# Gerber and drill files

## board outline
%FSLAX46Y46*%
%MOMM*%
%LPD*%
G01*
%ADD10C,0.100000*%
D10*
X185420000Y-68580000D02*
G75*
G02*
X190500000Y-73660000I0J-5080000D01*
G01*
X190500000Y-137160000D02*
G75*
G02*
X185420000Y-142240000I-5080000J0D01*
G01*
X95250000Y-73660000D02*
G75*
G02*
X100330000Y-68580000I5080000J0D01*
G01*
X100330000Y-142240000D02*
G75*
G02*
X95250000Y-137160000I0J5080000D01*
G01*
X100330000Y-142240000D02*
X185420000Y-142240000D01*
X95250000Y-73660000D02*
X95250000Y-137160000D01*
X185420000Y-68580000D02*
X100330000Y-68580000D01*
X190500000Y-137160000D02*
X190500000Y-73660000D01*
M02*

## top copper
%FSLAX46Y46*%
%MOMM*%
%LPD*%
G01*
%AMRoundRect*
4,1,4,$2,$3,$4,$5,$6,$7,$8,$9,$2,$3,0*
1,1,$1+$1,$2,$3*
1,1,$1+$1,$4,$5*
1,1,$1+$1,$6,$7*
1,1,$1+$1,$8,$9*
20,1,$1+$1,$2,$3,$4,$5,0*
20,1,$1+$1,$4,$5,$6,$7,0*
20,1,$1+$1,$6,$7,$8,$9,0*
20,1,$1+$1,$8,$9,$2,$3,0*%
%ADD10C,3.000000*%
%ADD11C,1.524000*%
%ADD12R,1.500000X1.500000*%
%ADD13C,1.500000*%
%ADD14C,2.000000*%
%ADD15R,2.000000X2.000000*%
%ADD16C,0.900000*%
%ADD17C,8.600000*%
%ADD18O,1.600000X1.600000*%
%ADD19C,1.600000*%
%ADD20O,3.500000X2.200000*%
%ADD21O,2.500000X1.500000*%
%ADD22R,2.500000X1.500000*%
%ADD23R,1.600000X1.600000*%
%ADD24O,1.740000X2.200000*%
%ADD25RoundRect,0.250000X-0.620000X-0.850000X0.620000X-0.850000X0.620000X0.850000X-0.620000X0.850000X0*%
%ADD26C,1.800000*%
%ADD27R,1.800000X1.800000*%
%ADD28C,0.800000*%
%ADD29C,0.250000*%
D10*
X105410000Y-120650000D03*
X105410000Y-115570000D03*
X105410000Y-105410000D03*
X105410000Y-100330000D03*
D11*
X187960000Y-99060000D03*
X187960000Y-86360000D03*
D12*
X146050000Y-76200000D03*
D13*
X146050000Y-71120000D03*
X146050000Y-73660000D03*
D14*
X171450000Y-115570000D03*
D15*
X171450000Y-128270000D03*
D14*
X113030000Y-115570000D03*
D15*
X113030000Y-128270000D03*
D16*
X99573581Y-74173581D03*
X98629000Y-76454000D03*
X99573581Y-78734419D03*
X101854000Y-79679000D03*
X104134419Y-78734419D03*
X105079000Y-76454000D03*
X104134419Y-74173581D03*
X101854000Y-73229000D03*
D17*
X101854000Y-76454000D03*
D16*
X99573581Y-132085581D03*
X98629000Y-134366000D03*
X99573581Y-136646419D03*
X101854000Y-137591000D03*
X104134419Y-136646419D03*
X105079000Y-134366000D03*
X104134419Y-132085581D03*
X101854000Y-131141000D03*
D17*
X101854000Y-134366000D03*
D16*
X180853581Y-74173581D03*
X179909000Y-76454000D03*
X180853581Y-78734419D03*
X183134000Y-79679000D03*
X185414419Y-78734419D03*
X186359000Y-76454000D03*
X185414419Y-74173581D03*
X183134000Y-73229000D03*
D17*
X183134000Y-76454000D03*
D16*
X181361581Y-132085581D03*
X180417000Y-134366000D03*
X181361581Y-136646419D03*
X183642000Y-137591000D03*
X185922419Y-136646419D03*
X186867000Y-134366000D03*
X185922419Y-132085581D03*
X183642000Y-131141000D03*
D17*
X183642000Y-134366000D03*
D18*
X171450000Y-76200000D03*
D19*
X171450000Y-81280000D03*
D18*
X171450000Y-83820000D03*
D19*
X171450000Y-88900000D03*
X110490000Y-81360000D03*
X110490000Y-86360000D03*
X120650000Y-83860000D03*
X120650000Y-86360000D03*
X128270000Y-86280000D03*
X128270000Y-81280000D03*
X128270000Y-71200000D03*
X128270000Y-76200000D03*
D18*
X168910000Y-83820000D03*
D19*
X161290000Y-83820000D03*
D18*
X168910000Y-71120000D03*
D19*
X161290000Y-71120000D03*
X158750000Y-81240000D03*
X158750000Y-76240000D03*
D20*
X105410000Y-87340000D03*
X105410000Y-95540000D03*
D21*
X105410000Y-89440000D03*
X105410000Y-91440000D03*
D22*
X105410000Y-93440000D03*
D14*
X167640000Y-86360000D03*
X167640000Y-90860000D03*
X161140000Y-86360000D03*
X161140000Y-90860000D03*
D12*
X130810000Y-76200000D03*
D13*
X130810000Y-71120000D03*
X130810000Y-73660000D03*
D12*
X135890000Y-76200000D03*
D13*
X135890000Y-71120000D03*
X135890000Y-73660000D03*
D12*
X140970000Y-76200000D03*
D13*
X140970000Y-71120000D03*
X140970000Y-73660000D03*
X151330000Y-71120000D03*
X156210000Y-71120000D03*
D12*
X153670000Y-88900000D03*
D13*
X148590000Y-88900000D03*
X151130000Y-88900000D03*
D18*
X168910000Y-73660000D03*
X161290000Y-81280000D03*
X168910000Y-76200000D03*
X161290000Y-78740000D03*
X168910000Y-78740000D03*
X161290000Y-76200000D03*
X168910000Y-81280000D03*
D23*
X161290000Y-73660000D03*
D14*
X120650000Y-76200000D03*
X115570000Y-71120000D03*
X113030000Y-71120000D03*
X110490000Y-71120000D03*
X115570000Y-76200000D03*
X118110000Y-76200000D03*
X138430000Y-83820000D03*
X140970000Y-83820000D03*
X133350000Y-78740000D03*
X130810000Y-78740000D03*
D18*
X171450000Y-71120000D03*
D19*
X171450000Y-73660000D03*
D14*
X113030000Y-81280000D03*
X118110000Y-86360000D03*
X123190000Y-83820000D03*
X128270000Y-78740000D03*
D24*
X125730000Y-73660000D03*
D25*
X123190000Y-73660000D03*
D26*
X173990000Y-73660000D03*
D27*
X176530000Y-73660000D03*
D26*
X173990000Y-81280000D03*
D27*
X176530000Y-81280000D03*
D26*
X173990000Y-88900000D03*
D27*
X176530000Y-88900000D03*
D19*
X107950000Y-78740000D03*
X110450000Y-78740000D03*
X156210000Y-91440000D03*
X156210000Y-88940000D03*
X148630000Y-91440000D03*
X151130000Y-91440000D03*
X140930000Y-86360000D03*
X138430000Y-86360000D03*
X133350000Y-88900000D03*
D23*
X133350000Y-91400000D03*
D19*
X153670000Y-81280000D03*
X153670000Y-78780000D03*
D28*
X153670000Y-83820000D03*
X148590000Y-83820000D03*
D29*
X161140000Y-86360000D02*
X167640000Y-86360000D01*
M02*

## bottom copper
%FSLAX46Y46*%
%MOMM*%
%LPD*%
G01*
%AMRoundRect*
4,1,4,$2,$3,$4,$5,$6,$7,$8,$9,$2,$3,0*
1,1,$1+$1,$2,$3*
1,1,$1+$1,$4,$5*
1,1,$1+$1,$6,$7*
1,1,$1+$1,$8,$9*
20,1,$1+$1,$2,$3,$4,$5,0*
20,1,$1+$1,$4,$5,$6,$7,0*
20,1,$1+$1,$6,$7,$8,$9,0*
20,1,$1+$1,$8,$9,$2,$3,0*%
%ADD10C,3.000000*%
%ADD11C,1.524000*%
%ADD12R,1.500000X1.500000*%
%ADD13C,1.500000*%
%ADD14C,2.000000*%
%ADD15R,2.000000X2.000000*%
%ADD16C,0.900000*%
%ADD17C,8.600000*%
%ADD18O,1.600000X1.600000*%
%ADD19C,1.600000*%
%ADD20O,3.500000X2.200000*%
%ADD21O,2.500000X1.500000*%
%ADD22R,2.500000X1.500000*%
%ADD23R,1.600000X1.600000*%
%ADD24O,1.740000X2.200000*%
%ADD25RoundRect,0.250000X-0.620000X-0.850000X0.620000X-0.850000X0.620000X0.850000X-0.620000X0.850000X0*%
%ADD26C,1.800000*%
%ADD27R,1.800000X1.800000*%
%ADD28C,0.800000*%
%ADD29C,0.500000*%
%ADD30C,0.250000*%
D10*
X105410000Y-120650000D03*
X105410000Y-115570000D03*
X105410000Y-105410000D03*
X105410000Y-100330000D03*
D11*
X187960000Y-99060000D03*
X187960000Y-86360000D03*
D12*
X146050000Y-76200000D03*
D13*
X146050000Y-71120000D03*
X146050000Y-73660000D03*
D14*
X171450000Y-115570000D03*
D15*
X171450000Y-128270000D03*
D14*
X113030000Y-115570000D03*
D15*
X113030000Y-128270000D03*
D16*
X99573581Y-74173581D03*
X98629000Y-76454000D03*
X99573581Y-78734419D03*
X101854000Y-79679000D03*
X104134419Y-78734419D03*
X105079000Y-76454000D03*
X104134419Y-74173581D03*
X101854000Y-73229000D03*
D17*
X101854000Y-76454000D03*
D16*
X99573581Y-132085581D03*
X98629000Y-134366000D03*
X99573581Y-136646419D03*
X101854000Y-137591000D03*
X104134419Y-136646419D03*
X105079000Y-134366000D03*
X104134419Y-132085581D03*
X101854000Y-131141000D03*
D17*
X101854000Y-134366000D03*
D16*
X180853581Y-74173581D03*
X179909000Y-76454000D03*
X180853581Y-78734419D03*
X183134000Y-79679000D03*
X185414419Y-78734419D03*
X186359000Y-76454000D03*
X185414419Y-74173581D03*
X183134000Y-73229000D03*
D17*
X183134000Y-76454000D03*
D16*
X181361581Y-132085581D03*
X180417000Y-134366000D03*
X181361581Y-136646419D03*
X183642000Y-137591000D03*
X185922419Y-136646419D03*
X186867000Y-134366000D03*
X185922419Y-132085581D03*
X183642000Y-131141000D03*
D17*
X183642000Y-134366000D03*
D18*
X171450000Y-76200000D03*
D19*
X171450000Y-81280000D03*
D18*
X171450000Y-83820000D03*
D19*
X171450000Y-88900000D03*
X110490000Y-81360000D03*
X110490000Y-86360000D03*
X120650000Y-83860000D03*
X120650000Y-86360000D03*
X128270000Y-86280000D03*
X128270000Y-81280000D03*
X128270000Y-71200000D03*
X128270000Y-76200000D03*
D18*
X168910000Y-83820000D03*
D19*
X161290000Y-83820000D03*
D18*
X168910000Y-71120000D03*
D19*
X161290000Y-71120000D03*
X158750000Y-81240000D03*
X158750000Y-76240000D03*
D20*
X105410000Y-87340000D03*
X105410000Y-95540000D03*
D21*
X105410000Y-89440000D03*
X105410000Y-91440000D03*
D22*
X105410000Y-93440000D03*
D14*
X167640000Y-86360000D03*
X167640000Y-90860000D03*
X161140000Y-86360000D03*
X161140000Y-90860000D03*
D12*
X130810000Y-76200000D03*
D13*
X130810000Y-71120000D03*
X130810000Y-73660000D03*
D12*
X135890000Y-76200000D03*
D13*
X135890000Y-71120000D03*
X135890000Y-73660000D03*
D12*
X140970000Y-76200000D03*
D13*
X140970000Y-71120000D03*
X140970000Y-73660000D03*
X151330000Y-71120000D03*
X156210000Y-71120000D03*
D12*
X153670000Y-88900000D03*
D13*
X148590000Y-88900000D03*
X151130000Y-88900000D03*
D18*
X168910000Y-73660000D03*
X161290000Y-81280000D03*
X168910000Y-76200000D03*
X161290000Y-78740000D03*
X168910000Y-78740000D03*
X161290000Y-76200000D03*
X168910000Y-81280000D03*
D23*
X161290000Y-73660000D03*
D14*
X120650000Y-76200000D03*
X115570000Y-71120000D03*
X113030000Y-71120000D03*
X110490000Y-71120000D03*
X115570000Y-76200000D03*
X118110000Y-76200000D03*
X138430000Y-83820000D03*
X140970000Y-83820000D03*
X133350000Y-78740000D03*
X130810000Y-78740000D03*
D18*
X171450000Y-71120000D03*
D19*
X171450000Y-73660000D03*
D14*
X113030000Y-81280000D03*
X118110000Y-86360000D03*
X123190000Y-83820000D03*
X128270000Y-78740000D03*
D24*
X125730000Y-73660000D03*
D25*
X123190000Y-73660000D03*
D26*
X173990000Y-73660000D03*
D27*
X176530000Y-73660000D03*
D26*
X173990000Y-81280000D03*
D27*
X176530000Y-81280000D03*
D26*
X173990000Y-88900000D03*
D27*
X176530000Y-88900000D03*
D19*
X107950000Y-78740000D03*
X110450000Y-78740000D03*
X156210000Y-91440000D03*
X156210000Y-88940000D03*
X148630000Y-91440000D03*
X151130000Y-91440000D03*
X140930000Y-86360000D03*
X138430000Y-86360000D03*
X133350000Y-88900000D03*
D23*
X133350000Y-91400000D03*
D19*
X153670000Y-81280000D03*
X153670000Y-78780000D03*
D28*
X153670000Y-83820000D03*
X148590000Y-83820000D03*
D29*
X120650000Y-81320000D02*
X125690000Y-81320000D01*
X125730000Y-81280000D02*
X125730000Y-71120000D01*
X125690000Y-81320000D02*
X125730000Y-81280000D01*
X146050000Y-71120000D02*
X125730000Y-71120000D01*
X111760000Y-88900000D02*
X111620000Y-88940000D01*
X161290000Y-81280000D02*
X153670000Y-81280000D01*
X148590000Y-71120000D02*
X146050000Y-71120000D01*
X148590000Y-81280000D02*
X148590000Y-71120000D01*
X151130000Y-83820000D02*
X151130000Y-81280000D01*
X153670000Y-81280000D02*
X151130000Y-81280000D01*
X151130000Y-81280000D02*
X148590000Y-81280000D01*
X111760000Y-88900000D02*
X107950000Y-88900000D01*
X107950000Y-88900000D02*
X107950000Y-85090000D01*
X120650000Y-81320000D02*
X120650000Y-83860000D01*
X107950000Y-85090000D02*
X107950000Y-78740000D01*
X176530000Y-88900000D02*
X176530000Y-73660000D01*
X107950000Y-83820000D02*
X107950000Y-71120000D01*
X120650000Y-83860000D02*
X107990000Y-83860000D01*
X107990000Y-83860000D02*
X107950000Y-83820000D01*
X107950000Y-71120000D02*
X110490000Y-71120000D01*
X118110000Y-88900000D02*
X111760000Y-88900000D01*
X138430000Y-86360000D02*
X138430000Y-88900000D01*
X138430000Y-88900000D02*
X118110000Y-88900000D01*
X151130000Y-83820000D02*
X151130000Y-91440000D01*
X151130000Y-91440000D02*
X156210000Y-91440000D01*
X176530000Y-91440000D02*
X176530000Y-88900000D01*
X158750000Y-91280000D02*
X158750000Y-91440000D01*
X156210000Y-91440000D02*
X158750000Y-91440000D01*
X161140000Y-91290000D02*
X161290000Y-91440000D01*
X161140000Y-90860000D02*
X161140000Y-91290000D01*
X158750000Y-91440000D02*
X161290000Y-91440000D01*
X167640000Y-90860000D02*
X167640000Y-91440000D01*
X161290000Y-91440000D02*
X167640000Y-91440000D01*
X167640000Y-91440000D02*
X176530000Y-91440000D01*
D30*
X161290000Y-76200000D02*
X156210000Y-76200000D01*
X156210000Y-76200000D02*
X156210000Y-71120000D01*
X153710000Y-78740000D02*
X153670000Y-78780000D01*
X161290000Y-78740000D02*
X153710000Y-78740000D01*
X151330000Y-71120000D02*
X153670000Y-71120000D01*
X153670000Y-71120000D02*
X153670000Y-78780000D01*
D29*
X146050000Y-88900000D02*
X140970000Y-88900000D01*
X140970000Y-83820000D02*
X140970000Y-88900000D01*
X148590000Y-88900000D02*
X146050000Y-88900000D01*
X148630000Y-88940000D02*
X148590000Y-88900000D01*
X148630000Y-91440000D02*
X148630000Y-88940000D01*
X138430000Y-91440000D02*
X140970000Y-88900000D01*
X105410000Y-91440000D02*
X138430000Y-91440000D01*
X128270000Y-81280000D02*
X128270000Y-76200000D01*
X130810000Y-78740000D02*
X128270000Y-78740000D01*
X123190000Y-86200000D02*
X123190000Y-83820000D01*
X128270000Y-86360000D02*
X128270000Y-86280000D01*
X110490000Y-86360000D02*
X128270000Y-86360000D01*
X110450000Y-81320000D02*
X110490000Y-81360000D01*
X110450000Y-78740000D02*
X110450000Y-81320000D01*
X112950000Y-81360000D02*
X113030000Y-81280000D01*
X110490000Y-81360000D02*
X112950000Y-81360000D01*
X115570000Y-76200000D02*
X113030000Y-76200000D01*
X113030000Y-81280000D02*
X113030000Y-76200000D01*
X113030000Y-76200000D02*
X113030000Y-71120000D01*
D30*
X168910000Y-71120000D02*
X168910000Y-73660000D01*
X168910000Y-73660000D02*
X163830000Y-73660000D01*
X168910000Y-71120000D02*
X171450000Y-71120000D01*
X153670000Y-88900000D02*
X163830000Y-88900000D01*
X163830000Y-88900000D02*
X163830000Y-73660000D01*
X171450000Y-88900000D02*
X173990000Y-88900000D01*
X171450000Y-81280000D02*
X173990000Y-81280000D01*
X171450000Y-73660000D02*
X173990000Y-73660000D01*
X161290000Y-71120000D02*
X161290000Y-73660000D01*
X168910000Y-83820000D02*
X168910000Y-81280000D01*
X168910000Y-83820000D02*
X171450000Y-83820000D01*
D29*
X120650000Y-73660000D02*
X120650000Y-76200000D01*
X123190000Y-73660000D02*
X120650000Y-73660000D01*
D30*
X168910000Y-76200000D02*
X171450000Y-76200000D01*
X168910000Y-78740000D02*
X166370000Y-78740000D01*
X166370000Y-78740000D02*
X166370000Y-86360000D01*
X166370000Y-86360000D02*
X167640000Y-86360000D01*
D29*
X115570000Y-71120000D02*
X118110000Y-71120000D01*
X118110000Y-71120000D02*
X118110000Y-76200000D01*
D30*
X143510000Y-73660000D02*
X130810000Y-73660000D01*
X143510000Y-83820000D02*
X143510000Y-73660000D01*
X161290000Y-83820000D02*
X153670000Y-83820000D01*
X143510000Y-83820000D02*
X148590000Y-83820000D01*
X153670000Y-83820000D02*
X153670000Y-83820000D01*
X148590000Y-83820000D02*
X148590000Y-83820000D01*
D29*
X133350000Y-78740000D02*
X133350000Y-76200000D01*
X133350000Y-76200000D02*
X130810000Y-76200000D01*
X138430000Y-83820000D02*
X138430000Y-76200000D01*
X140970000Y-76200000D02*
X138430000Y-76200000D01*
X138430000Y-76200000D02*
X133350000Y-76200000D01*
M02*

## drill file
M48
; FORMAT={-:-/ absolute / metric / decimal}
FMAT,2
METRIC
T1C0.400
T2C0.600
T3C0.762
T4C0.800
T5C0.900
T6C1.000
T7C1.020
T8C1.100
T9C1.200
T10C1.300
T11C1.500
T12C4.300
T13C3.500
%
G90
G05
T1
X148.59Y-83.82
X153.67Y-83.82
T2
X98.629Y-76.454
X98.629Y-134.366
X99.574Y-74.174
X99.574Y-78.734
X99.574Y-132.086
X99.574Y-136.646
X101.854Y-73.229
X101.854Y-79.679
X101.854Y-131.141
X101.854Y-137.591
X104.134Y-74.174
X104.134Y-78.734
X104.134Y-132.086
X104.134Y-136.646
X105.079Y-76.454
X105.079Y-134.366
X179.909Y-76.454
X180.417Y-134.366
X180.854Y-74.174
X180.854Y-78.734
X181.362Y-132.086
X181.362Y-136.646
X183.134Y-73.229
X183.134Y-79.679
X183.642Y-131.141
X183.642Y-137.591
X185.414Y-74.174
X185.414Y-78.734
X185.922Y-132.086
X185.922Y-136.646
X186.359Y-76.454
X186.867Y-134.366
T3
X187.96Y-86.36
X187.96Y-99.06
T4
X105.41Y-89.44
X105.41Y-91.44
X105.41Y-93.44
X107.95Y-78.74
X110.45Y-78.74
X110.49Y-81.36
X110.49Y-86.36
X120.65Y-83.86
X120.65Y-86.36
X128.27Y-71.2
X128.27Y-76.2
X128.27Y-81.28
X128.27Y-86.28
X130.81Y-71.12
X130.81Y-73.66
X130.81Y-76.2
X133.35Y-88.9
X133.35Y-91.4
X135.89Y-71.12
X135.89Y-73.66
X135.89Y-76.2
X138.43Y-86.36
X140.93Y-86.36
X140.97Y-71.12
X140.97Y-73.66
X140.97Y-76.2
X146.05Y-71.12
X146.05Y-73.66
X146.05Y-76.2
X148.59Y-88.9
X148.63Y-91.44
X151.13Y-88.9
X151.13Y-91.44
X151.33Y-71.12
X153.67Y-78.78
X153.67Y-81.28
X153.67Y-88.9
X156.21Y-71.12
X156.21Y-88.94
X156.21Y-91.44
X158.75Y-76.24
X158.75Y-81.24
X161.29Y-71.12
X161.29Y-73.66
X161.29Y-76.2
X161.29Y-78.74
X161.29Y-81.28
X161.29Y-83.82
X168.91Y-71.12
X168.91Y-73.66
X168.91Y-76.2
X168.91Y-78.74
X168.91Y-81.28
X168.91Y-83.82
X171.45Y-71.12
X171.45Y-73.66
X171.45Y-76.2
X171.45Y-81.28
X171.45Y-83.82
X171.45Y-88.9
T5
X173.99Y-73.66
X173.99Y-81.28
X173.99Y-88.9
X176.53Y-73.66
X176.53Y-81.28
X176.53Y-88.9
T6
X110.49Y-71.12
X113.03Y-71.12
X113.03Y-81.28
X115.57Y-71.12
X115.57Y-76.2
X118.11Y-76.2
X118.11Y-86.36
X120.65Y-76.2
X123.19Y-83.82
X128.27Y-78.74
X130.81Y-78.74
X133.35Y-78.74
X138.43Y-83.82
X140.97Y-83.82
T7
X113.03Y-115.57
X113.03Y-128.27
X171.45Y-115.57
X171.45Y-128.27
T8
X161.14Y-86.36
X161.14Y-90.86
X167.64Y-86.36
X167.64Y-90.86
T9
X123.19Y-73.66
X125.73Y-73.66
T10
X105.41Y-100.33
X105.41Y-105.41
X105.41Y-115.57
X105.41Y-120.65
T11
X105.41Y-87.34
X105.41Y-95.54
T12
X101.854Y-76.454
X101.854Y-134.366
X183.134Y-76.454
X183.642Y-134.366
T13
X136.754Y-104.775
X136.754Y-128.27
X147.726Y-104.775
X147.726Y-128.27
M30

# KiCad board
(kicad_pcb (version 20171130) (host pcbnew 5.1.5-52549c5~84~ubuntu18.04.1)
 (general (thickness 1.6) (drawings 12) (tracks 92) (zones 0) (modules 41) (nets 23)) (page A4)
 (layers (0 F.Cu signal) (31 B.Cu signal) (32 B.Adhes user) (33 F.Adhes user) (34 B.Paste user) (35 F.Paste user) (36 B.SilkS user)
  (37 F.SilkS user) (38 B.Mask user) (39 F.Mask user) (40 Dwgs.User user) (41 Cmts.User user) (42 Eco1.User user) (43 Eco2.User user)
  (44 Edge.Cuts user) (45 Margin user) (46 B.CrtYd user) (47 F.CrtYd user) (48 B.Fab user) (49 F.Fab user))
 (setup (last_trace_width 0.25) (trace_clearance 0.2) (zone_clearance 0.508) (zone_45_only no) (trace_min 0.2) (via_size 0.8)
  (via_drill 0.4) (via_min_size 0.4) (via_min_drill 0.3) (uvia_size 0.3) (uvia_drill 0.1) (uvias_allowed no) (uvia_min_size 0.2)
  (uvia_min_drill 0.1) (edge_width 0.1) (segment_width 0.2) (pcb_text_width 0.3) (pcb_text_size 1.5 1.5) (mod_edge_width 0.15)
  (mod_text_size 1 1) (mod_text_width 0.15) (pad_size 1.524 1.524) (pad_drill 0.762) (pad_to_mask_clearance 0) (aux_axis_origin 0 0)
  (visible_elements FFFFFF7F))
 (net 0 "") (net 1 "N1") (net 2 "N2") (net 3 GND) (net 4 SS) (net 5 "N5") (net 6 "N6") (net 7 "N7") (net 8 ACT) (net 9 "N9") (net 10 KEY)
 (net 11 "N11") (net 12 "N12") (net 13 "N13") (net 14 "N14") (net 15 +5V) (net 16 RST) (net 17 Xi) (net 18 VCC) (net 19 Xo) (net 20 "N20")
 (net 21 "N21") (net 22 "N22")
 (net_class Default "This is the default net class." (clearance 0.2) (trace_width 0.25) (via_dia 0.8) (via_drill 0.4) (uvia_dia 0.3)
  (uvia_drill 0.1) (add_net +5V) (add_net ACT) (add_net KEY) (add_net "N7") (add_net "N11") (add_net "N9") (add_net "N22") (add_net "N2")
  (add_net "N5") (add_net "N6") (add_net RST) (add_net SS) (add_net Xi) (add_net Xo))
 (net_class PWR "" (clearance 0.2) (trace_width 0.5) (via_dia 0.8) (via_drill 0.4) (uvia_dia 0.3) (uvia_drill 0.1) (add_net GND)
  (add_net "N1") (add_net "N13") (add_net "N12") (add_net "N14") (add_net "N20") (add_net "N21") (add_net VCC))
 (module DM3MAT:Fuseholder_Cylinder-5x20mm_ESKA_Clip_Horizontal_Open (layer F.Cu) (at 111.76 110.49 270)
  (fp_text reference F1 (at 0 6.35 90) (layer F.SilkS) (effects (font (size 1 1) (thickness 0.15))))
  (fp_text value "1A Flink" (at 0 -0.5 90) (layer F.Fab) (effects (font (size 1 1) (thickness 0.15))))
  (pad 2 thru_hole circle (at 10.16 6.35 270) (size 3 3) (drill 1.3) (layers *.Cu *.Mask) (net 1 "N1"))
  (pad 2 thru_hole circle (at 5.08 6.35 270) (size 3 3) (drill 1.3) (layers *.Cu *.Mask) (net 1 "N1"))
  (pad 1 thru_hole circle (at -5.08 6.35 270) (size 3 3) (drill 1.3) (layers *.Cu *.Mask) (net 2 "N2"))
  (pad 1 thru_hole circle (at -10.16 6.35 270) (size 3 3) (drill 1.3) (layers *.Cu *.Mask) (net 2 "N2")))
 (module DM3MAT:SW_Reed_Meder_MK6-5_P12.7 (layer F.Cu) (at 187.96 92.71 270)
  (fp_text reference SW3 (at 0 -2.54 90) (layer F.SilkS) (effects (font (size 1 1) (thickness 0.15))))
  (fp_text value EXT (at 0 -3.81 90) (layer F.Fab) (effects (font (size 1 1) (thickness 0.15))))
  (pad 2 thru_hole circle (at 6.35 0 270) (size 1.524 1.524) (drill 0.762) (layers *.Cu *.Mask) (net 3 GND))
  (pad 1 thru_hole circle (at -6.35 0 270) (size 1.524 1.524) (drill 0.762) (layers *.Cu *.Mask) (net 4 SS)))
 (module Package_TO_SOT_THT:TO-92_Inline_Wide (layer F.Cu) (at 146.05 76.2 90)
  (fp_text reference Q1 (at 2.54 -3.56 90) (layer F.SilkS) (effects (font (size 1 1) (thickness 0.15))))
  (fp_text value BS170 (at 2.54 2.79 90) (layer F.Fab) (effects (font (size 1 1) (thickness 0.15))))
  (pad 1 thru_hole rect (at 0 0 180) (size 1.5 1.5) (drill 0.8) (layers *.Cu *.Mask) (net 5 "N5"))
  (pad 3 thru_hole circle (at 5.08 0 180) (size 1.5 1.5) (drill 0.8) (layers *.Cu *.Mask) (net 3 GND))
  (pad 2 thru_hole circle (at 2.54 0 180) (size 1.5 1.5) (drill 0.8) (layers *.Cu *.Mask) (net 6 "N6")))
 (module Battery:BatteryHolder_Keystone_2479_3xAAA (layer F.Cu) (at 171.45 128.27 180)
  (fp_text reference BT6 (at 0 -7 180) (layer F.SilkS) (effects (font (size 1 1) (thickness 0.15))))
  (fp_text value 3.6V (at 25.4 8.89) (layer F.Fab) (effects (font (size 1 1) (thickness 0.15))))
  (pad "" np_thru_hole circle (at 23.7236 0 180) (size 3.5 3.5) (drill 3.5) (layers *.Cu *.Mask))
  (pad "" np_thru_hole circle (at 23.7236 23.495 180) (size 3.5 3.5) (drill 3.5) (layers *.Cu *.Mask))
  (pad 2 thru_hole circle (at 0 12.7 180) (size 2 2) (drill 1.02) (layers *.Cu *.Mask) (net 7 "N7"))
  (pad 1 thru_hole rect (at 0 0 180) (size 2 2) (drill 1.02) (layers *.Cu *.Mask) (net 1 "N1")))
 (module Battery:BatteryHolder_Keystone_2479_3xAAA (layer B.Cu) (at 113.03 128.27)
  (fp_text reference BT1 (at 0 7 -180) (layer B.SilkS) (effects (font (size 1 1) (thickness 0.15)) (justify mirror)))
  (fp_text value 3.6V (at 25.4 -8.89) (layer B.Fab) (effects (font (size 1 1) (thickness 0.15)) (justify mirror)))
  (pad "" np_thru_hole circle (at 23.7236 0) (size 3.5 3.5) (drill 3.5) (layers *.Cu *.Mask))
  (pad "" np_thru_hole circle (at 23.7236 -23.495) (size 3.5 3.5) (drill 3.5) (layers *.Cu *.Mask))
  (pad 2 thru_hole circle (at 0 -12.7) (size 2 2) (drill 1.02) (layers *.Cu *.Mask) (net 3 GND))
  (pad 1 thru_hole rect (at 0 0) (size 2 2) (drill 1.02) (layers *.Cu *.Mask) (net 7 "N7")))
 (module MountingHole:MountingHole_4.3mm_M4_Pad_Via (layer F.Cu) (at 101.854 76.454 90)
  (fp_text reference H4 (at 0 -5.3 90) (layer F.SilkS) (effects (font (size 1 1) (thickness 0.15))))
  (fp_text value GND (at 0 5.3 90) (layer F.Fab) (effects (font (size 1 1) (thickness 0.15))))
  (pad 1 thru_hole circle (at 2.280419 -2.280419 90) (size 0.9 0.9) (drill 0.6) (layers *.Cu *.Mask) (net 3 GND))
  (pad 1 thru_hole circle (at 0 -3.225 90) (size 0.9 0.9) (drill 0.6) (layers *.Cu *.Mask) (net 3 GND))
  (pad 1 thru_hole circle (at -2.280419 -2.280419 90) (size 0.9 0.9) (drill 0.6) (layers *.Cu *.Mask) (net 3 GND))
  (pad 1 thru_hole circle (at -3.225 0 90) (size 0.9 0.9) (drill 0.6) (layers *.Cu *.Mask) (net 3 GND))
  (pad 1 thru_hole circle (at -2.280419 2.280419 90) (size 0.9 0.9) (drill 0.6) (layers *.Cu *.Mask) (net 3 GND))
  (pad 1 thru_hole circle (at 0 3.225 90) (size 0.9 0.9) (drill 0.6) (layers *.Cu *.Mask) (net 3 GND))
  (pad 1 thru_hole circle (at 2.280419 2.280419 90) (size 0.9 0.9) (drill 0.6) (layers *.Cu *.Mask) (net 3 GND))
  (pad 1 thru_hole circle (at 3.225 0 90) (size 0.9 0.9) (drill 0.6) (layers *.Cu *.Mask) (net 3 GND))
  (pad 1 thru_hole circle (at 0 0 90) (size 8.6 8.6) (drill 4.3) (layers *.Cu *.Mask) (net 3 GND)))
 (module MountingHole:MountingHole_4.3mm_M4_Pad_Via (layer F.Cu) (at 101.854 134.366 90)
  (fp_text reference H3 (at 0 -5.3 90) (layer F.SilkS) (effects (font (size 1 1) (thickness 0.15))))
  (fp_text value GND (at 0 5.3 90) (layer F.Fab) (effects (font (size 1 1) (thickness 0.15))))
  (pad 1 thru_hole circle (at 2.280419 -2.280419 90) (size 0.9 0.9) (drill 0.6) (layers *.Cu *.Mask) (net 3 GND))
  (pad 1 thru_hole circle (at 0 -3.225 90) (size 0.9 0.9) (drill 0.6) (layers *.Cu *.Mask) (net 3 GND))
  (pad 1 thru_hole circle (at -2.280419 -2.280419 90) (size 0.9 0.9) (drill 0.6) (layers *.Cu *.Mask) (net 3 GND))
  (pad 1 thru_hole circle (at -3.225 0 90) (size 0.9 0.9) (drill 0.6) (layers *.Cu *.Mask) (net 3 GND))
  (pad 1 thru_hole circle (at -2.280419 2.280419 90) (size 0.9 0.9) (drill 0.6) (layers *.Cu *.Mask) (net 3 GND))
  (pad 1 thru_hole circle (at 0 3.225 90) (size 0.9 0.9) (drill 0.6) (layers *.Cu *.Mask) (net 3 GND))
  (pad 1 thru_hole circle (at 2.280419 2.280419 90) (size 0.9 0.9) (drill 0.6) (layers *.Cu *.Mask) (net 3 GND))
  (pad 1 thru_hole circle (at 3.225 0 90) (size 0.9 0.9) (drill 0.6) (layers *.Cu *.Mask) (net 3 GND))
  (pad 1 thru_hole circle (at 0 0 90) (size 8.6 8.6) (drill 4.3) (layers *.Cu *.Mask) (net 3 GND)))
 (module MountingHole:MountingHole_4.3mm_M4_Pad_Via (layer F.Cu) (at 183.134 76.454 90)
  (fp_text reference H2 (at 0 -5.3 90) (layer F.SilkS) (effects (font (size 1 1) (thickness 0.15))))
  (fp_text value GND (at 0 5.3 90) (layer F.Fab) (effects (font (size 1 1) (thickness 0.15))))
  (pad 1 thru_hole circle (at 2.280419 -2.280419 90) (size 0.9 0.9) (drill 0.6) (layers *.Cu *.Mask) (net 3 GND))
  (pad 1 thru_hole circle (at 0 -3.225 90) (size 0.9 0.9) (drill 0.6) (layers *.Cu *.Mask) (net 3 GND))
  (pad 1 thru_hole circle (at -2.280419 -2.280419 90) (size 0.9 0.9) (drill 0.6) (layers *.Cu *.Mask) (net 3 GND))
  (pad 1 thru_hole circle (at -3.225 0 90) (size 0.9 0.9) (drill 0.6) (layers *.Cu *.Mask) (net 3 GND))
  (pad 1 thru_hole circle (at -2.280419 2.280419 90) (size 0.9 0.9) (drill 0.6) (layers *.Cu *.Mask) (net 3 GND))
  (pad 1 thru_hole circle (at 0 3.225 90) (size 0.9 0.9) (drill 0.6) (layers *.Cu *.Mask) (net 3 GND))
  (pad 1 thru_hole circle (at 2.280419 2.280419 90) (size 0.9 0.9) (drill 0.6) (layers *.Cu *.Mask) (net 3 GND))
  (pad 1 thru_hole circle (at 3.225 0 90) (size 0.9 0.9) (drill 0.6) (layers *.Cu *.Mask) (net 3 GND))
  (pad 1 thru_hole circle (at 0 0 90) (size 8.6 8.6) (drill 4.3) (layers *.Cu *.Mask) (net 3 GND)))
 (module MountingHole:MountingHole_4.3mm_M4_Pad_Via (layer F.Cu) (at 183.642 134.366 90)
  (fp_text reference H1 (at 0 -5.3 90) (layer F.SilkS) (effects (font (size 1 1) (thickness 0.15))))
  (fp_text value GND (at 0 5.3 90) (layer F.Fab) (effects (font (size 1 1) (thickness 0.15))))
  (pad 1 thru_hole circle (at 2.280419 -2.280419 90) (size 0.9 0.9) (drill 0.6) (layers *.Cu *.Mask) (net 3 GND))
  (pad 1 thru_hole circle (at 0 -3.225 90) (size 0.9 0.9) (drill 0.6) (layers *.Cu *.Mask) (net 3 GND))
  (pad 1 thru_hole circle (at -2.280419 -2.280419 90) (size 0.9 0.9) (drill 0.6) (layers *.Cu *.Mask) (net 3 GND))
  (pad 1 thru_hole circle (at -3.225 0 90) (size 0.9 0.9) (drill 0.6) (layers *.Cu *.Mask) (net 3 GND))
  (pad 1 thru_hole circle (at -2.280419 2.280419 90) (size 0.9 0.9) (drill 0.6) (layers *.Cu *.Mask) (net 3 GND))
  (pad 1 thru_hole circle (at 0 3.225 90) (size 0.9 0.9) (drill 0.6) (layers *.Cu *.Mask) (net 3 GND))
  (pad 1 thru_hole circle (at 2.280419 2.280419 90) (size 0.9 0.9) (drill 0.6) (layers *.Cu *.Mask) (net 3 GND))
  (pad 1 thru_hole circle (at 3.225 0 90) (size 0.9 0.9) (drill 0.6) (layers *.Cu *.Mask) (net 3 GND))
  (pad 1 thru_hole circle (at 0 0 90) (size 8.6 8.6) (drill 4.3) (layers *.Cu *.Mask) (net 3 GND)))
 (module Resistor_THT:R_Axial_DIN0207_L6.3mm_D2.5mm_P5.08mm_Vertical (layer F.Cu) (at 171.45 81.28 90)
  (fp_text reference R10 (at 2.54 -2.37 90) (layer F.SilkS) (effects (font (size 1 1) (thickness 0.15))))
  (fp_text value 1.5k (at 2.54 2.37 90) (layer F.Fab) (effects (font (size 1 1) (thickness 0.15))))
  (pad 2 thru_hole oval (at 5.08 0 90) (size 1.6 1.6) (drill 0.8) (layers *.Cu *.Mask) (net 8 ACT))
  (pad 1 thru_hole circle (at 0 0 90) (size 1.6 1.6) (drill 0.8) (layers *.Cu *.Mask) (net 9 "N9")))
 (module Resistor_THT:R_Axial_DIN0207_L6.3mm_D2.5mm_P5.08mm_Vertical (layer F.Cu) (at 171.45 88.9 90)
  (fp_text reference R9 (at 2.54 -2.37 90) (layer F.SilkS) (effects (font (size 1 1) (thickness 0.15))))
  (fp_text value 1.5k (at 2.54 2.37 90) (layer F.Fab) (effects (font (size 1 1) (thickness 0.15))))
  (pad 2 thru_hole oval (at 5.08 0 90) (size 1.6 1.6) (drill 0.8) (layers *.Cu *.Mask) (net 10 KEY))
  (pad 1 thru_hole circle (at 0 0 90) (size 1.6 1.6) (drill 0.8) (layers *.Cu *.Mask) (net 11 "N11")))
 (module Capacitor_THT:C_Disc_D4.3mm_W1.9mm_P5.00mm (layer F.Cu) (at 110.49 86.36 90)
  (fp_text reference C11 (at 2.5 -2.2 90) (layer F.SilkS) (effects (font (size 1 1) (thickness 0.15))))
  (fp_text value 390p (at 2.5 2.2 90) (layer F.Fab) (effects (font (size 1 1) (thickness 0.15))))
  (pad 2 thru_hole circle (at 5 0 90) (size 1.6 1.6) (drill 0.8) (layers *.Cu *.Mask) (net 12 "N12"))
  (pad 1 thru_hole circle (at 0 0 90) (size 1.6 1.6) (drill 0.8) (layers *.Cu *.Mask) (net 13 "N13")))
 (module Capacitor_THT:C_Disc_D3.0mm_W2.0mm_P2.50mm (layer F.Cu) (at 120.65 86.36 90)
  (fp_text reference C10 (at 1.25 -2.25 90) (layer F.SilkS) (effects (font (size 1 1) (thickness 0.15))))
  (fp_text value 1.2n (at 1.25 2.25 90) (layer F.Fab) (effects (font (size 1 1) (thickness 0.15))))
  (pad 2 thru_hole circle (at 2.5 0 90) (size 1.6 1.6) (drill 0.8) (layers *.Cu *.Mask) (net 3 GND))
  (pad 1 thru_hole circle (at 0 0 90) (size 1.6 1.6) (drill 0.8) (layers *.Cu *.Mask) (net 13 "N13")))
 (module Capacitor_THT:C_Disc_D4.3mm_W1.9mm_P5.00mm (layer F.Cu) (at 128.27 81.28 270)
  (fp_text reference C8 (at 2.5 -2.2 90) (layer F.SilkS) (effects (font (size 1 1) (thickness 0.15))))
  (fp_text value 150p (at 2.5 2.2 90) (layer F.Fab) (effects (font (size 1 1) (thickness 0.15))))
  (pad 2 thru_hole circle (at 5 0 270) (size 1.6 1.6) (drill 0.8) (layers *.Cu *.Mask) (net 13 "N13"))
  (pad 1 thru_hole circle (at 0 0 270) (size 1.6 1.6) (drill 0.8) (layers *.Cu *.Mask) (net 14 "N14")))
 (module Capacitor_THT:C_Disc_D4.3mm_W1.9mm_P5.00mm (layer F.Cu) (at 128.27 76.2 90)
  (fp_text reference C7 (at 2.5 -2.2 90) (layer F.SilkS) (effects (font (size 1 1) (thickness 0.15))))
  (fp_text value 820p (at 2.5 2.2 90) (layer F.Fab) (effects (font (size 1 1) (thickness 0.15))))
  (pad 2 thru_hole circle (at 5 0 90) (size 1.6 1.6) (drill 0.8) (layers *.Cu *.Mask) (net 3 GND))
  (pad 1 thru_hole circle (at 0 0 90) (size 1.6 1.6) (drill 0.8) (layers *.Cu *.Mask) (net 14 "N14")))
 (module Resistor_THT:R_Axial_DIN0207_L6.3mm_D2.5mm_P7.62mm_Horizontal (layer F.Cu) (at 161.29 83.82)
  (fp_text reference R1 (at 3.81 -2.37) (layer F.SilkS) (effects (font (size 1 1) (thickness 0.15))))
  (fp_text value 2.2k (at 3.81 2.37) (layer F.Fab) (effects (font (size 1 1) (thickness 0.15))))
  (pad 2 thru_hole oval (at 7.62 0) (size 1.6 1.6) (drill 0.8) (layers *.Cu *.Mask) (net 10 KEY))
  (pad 1 thru_hole circle (at 0 0) (size 1.6 1.6) (drill 0.8) (layers *.Cu *.Mask) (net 6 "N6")))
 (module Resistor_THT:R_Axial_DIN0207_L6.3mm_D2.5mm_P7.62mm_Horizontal (layer F.Cu) (at 161.29 71.12)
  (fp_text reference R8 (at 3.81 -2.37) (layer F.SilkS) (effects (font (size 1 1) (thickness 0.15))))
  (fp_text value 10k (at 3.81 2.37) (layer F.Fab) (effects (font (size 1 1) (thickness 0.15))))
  (pad 2 thru_hole oval (at 7.62 0) (size 1.6 1.6) (drill 0.8) (layers *.Cu *.Mask) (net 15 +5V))
  (pad 1 thru_hole circle (at 0 0) (size 1.6 1.6) (drill 0.8) (layers *.Cu *.Mask) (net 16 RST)))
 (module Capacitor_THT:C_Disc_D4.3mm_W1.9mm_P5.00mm (layer F.Cu) (at 158.75 76.24 270)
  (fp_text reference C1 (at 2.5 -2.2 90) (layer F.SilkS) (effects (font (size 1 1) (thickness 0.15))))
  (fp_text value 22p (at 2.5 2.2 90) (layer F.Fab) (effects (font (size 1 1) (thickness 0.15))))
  (pad 2 thru_hole circle (at 5 0 270) (size 1.6 1.6) (drill 0.8) (layers *.Cu *.Mask) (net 3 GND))
  (pad 1 thru_hole circle (at 0 0 270) (size 1.6 1.6) (drill 0.8) (layers *.Cu *.Mask) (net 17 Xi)))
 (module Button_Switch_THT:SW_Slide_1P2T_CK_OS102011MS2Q (layer F.Cu) (at 105.41 93.44 90)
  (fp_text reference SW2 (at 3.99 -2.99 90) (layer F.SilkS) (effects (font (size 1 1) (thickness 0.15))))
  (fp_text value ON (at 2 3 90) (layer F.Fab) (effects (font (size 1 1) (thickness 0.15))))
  (pad "" thru_hole oval (at 6.1 0 90) (size 2.2 3.5) (drill 1.5) (layers *.Cu *.Mask))
  (pad "" thru_hole oval (at -2.1 0 90) (size 2.2 3.5) (drill 1.5) (layers *.Cu *.Mask))
  (pad 3 thru_hole oval (at 4 0 90) (size 1.5 2.5) (drill 0.8) (layers *.Cu *.Mask))
  (pad 2 thru_hole oval (at 2 0 90) (size 1.5 2.5) (drill 0.8) (layers *.Cu *.Mask) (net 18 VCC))
  (pad 1 thru_hole rect (at 0 0 90) (size 1.5 2.5) (drill 0.8) (layers *.Cu *.Mask) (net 2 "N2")))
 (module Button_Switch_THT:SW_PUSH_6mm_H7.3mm (layer F.Cu) (at 161.14 86.36)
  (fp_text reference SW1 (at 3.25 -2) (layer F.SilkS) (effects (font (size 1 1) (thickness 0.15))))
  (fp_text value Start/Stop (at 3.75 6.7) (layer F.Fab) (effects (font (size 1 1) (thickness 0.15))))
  (pad 1 thru_hole circle (at 6.5 0 90) (size 2 2) (drill 1.1) (layers *.Cu *.Mask) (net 4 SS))
  (pad 2 thru_hole circle (at 6.5 4.5 90) (size 2 2) (drill 1.1) (layers *.Cu *.Mask) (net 3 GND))
  (pad 1 thru_hole circle (at 0 0 90) (size 2 2) (drill 1.1) (layers *.Cu *.Mask) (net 4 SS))
  (pad 2 thru_hole circle (at 0 4.5 90) (size 2 2) (drill 1.1) (layers *.Cu *.Mask) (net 3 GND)))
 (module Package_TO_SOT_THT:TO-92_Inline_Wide (layer F.Cu) (at 130.81 76.2 90)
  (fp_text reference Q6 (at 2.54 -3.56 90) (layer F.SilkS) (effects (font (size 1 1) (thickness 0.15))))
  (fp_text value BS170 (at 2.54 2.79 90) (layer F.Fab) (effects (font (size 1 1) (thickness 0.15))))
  (pad 1 thru_hole rect (at 0 0 180) (size 1.5 1.5) (drill 0.8) (layers *.Cu *.Mask) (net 5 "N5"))
  (pad 3 thru_hole circle (at 5.08 0 180) (size 1.5 1.5) (drill 0.8) (layers *.Cu *.Mask) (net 3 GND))
  (pad 2 thru_hole circle (at 2.54 0 180) (size 1.5 1.5) (drill 0.8) (layers *.Cu *.Mask) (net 6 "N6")))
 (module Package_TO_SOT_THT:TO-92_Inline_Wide (layer F.Cu) (at 135.89 76.2 90)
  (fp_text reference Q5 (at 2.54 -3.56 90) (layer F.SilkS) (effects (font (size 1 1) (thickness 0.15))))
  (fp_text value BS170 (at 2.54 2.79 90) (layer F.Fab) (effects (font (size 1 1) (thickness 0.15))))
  (pad 1 thru_hole rect (at 0 0 180) (size 1.5 1.5) (drill 0.8) (layers *.Cu *.Mask) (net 5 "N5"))
  (pad 3 thru_hole circle (at 5.08 0 180) (size 1.5 1.5) (drill 0.8) (layers *.Cu *.Mask) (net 3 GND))
  (pad 2 thru_hole circle (at 2.54 0 180) (size 1.5 1.5) (drill 0.8) (layers *.Cu *.Mask) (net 6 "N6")))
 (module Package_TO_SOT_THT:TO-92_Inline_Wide (layer F.Cu) (at 140.97 76.2 90)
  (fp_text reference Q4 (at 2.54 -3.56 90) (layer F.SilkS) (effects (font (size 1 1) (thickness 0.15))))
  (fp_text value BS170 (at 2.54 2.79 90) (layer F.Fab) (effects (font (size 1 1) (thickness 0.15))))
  (pad 1 thru_hole rect (at 0 0 180) (size 1.5 1.5) (drill 0.8) (layers *.Cu *.Mask) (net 5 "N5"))
  (pad 3 thru_hole circle (at 5.08 0 180) (size 1.5 1.5) (drill 0.8) (layers *.Cu *.Mask) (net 3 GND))
  (pad 2 thru_hole circle (at 2.54 0 180) (size 1.5 1.5) (drill 0.8) (layers *.Cu *.Mask) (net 6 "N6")))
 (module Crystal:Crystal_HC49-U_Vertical (layer F.Cu) (at 156.21 71.12 180)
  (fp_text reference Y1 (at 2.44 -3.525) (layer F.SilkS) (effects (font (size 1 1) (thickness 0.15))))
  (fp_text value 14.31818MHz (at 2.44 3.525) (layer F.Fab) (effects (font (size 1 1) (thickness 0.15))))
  (pad 2 thru_hole circle (at 4.88 0 180) (size 1.5 1.5) (drill 0.8) (layers *.Cu *.Mask) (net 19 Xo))
  (pad 1 thru_hole circle (at 0 0 180) (size 1.5 1.5) (drill 0.8) (layers *.Cu *.Mask) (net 17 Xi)))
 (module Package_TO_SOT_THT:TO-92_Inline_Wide (layer F.Cu) (at 153.67 88.9 180)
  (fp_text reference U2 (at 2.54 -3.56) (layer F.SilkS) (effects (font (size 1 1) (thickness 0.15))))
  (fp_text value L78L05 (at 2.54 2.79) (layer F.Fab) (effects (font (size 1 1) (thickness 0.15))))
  (pad 1 thru_hole rect (at 0 0 270) (size 1.5 1.5) (drill 0.8) (layers *.Cu *.Mask) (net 15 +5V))
  (pad 3 thru_hole circle (at 5.08 0 270) (size 1.5 1.5) (drill 0.8) (layers *.Cu *.Mask) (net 18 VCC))
  (pad 2 thru_hole circle (at 2.54 0 270) (size 1.5 1.5) (drill 0.8) (layers *.Cu *.Mask) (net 3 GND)))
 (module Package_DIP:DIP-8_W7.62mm (layer F.Cu) (at 161.29 73.66)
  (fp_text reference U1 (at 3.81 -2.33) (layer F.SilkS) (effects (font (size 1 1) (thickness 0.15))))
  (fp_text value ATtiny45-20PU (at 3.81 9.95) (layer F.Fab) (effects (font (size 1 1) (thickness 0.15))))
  (pad 8 thru_hole oval (at 7.62 0) (size 1.6 1.6) (drill 0.8) (layers *.Cu *.Mask) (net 15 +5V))
  (pad 4 thru_hole oval (at 0 7.62) (size 1.6 1.6) (drill 0.8) (layers *.Cu *.Mask) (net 3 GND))
  (pad 7 thru_hole oval (at 7.62 2.54) (size 1.6 1.6) (drill 0.8) (layers *.Cu *.Mask) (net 8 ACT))
  (pad 3 thru_hole oval (at 0 5.08) (size 1.6 1.6) (drill 0.8) (layers *.Cu *.Mask) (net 19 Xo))
  (pad 6 thru_hole oval (at 7.62 5.08) (size 1.6 1.6) (drill 0.8) (layers *.Cu *.Mask) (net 4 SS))
  (pad 2 thru_hole oval (at 0 2.54) (size 1.6 1.6) (drill 0.8) (layers *.Cu *.Mask) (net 17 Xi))
  (pad 5 thru_hole oval (at 7.62 7.62) (size 1.6 1.6) (drill 0.8) (layers *.Cu *.Mask) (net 10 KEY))
  (pad 1 thru_hole rect (at 0 0) (size 1.6 1.6) (drill 0.8) (layers *.Cu *.Mask) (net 16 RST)))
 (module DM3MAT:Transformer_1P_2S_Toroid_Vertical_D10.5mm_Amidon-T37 (layer F.Cu) (at 115.57 71.12)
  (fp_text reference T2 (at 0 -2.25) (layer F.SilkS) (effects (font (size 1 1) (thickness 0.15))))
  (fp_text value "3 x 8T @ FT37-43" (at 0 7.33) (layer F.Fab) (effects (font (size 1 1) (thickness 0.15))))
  (pad 6 thru_hole circle (at 5.08 5.08) (size 2 2) (drill 1) (layers *.Cu *.Mask) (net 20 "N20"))
  (pad 5 thru_hole circle (at 0 0) (size 2 2) (drill 1) (layers *.Cu *.Mask) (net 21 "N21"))
  (pad 3 thru_hole circle (at -2.54 0) (size 2 2) (drill 1) (layers *.Cu *.Mask) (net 12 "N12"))
  (pad 1 thru_hole circle (at -5.08 0) (size 2 2) (drill 1) (layers *.Cu *.Mask) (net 3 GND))
  (pad 2 thru_hole circle (at 0 5.08) (size 2 2) (drill 1) (layers *.Cu *.Mask) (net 12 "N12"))
  (pad 4 thru_hole circle (at 2.54 5.08) (size 2 2) (drill 1) (layers *.Cu *.Mask) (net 21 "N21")))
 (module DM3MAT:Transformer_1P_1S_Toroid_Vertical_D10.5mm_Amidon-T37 (layer F.Cu) (at 135.89 83.82 180)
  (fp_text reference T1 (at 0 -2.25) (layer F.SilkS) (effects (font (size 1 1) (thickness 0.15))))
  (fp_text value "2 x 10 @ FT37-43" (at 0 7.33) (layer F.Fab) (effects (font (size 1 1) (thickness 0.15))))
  (pad 4 thru_hole circle (at -2.54 0 180) (size 2 2) (drill 1) (layers *.Cu *.Mask) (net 5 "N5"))
  (pad 1 thru_hole circle (at -5.08 0 180) (size 2 2) (drill 1) (layers *.Cu *.Mask) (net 18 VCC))
  (pad 2 thru_hole circle (at 2.54 5.08 180) (size 2 2) (drill 1) (layers *.Cu *.Mask) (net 5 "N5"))
  (pad 3 thru_hole circle (at 5.08 5.08 180) (size 2 2) (drill 1) (layers *.Cu *.Mask) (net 14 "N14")))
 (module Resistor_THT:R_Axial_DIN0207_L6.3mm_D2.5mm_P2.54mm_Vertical (layer F.Cu) (at 171.45 73.66 90)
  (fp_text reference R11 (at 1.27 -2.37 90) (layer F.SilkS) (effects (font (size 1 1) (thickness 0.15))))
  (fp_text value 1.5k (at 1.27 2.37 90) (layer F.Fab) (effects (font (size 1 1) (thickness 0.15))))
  (pad 2 thru_hole oval (at 2.54 0 90) (size 1.6 1.6) (drill 0.8) (layers *.Cu *.Mask) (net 15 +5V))
  (pad 1 thru_hole circle (at 0 0 90) (size 1.6 1.6) (drill 0.8) (layers *.Cu *.Mask) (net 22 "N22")))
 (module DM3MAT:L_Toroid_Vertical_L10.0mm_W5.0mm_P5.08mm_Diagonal (layer F.Cu) (at 115.57 86.36 180)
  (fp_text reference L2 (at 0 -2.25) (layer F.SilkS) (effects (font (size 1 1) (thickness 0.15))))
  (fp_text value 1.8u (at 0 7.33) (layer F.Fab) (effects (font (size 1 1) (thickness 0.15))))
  (pad 2 thru_hole circle (at 2.54 5.08 180) (size 2 2) (drill 1) (layers *.Cu *.Mask) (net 12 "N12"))
  (pad 1 thru_hole circle (at -2.54 0 180) (size 2 2) (drill 1) (layers *.Cu *.Mask) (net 13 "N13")))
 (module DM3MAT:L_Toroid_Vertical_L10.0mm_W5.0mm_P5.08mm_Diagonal (layer F.Cu) (at 128.27 81.28 270)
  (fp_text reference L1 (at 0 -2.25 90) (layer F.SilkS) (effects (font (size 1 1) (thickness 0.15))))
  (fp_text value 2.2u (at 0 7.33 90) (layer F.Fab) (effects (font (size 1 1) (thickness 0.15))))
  (pad 2 thru_hole circle (at 2.54 5.08 270) (size 2 2) (drill 1) (layers *.Cu *.Mask) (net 13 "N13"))
  (pad 1 thru_hole circle (at -2.54 0 270) (size 2 2) (drill 1) (layers *.Cu *.Mask) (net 14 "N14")))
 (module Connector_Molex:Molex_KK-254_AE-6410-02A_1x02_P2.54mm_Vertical (layer F.Cu) (at 123.19 73.66)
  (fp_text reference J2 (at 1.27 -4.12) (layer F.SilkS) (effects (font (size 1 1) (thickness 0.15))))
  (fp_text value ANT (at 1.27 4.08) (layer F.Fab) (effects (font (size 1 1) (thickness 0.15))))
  (pad 2 thru_hole oval (at 2.54 0) (size 1.74 2.2) (drill 1.2) (layers *.Cu *.Mask) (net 3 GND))
  (pad 1 thru_hole roundrect (at 0 0) (size 1.74 2.2) (drill 1.2) (layers *.Cu *.Mask) (roundrect_rratio 0.143678) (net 20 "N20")))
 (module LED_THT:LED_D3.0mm (layer F.Cu) (at 176.53 73.66 180)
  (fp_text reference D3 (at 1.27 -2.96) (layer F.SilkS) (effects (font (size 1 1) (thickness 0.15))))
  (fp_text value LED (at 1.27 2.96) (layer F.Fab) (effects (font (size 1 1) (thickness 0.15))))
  (pad 2 thru_hole circle (at 2.54 0 180) (size 1.8 1.8) (drill 0.9) (layers *.Cu *.Mask) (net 22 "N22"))
  (pad 1 thru_hole rect (at 0 0 180) (size 1.8 1.8) (drill 0.9) (layers *.Cu *.Mask) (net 3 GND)))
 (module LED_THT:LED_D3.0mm (layer F.Cu) (at 176.53 81.28 180)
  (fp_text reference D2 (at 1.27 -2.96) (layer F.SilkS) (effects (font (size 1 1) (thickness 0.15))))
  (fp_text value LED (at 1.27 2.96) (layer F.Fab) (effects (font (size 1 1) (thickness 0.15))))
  (pad 2 thru_hole circle (at 2.54 0 180) (size 1.8 1.8) (drill 0.9) (layers *.Cu *.Mask) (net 9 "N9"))
  (pad 1 thru_hole rect (at 0 0 180) (size 1.8 1.8) (drill 0.9) (layers *.Cu *.Mask) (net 3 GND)))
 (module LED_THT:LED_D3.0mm (layer F.Cu) (at 176.53 88.9 180)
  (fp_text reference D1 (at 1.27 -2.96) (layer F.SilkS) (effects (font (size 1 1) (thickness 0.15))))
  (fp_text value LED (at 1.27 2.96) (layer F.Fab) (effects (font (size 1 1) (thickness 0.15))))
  (pad 2 thru_hole circle (at 2.54 0 180) (size 1.8 1.8) (drill 0.9) (layers *.Cu *.Mask) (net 11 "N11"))
  (pad 1 thru_hole rect (at 0 0 180) (size 1.8 1.8) (drill 0.9) (layers *.Cu *.Mask) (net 3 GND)))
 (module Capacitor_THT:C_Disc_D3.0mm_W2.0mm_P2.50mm (layer F.Cu) (at 110.45 78.74 180)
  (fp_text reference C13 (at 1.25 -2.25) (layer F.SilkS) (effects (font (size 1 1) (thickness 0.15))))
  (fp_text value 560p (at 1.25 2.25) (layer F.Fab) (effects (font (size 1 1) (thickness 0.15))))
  (pad 2 thru_hole circle (at 2.5 0 180) (size 1.6 1.6) (drill 0.8) (layers *.Cu *.Mask) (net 3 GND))
  (pad 1 thru_hole circle (at 0 0 180) (size 1.6 1.6) (drill 0.8) (layers *.Cu *.Mask) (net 12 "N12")))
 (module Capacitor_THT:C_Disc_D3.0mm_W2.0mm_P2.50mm (layer F.Cu) (at 156.21 88.94 270)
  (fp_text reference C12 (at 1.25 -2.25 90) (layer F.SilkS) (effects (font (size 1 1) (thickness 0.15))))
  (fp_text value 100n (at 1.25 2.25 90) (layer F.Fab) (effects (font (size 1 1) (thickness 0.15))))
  (pad 2 thru_hole circle (at 2.5 0 270) (size 1.6 1.6) (drill 0.8) (layers *.Cu *.Mask) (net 3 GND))
  (pad 1 thru_hole circle (at 0 0 270) (size 1.6 1.6) (drill 0.8) (layers *.Cu *.Mask) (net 15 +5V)))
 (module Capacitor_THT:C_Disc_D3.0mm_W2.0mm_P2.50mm (layer F.Cu) (at 151.13 91.44 180)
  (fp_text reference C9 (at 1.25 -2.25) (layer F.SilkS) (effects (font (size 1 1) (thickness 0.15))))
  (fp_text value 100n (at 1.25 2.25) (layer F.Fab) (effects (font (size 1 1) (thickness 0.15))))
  (pad 2 thru_hole circle (at 2.5 0 180) (size 1.6 1.6) (drill 0.8) (layers *.Cu *.Mask) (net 18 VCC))
  (pad 1 thru_hole circle (at 0 0 180) (size 1.6 1.6) (drill 0.8) (layers *.Cu *.Mask) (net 3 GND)))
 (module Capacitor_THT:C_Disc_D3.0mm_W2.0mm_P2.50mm (layer F.Cu) (at 138.43 86.36)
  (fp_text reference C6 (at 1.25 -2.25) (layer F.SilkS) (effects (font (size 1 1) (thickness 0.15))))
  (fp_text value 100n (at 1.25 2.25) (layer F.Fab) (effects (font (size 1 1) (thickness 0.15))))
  (pad 2 thru_hole circle (at 2.5 0) (size 1.6 1.6) (drill 0.8) (layers *.Cu *.Mask) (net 18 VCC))
  (pad 1 thru_hole circle (at 0 0) (size 1.6 1.6) (drill 0.8) (layers *.Cu *.Mask) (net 3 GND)))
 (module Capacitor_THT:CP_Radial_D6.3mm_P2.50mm (layer F.Cu) (at 133.35 91.4 90)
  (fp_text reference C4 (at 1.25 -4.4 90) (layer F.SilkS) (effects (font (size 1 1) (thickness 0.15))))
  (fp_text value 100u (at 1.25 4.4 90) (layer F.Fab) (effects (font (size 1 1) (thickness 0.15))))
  (pad 2 thru_hole circle (at 2.5 0 90) (size 1.6 1.6) (drill 0.8) (layers *.Cu *.Mask) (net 3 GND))
  (pad 1 thru_hole rect (at 0 0 90) (size 1.6 1.6) (drill 0.8) (layers *.Cu *.Mask) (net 18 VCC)))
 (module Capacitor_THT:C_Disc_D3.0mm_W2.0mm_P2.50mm (layer F.Cu) (at 153.67 78.78 270)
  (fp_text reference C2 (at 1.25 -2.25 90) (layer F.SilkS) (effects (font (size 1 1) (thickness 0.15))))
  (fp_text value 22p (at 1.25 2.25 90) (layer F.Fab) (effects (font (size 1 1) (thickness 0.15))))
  (pad 2 thru_hole circle (at 2.5 0 270) (size 1.6 1.6) (drill 0.8) (layers *.Cu *.Mask) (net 3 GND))
  (pad 1 thru_hole circle (at 0 0 270) (size 1.6 1.6) (drill 0.8) (layers *.Cu *.Mask) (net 19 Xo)))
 (gr_arc (start 185.42 73.66) (end 190.5 73.66) (angle -90) (layer Edge.Cuts) (width 0.1))
 (gr_arc (start 185.42 137.16) (end 185.42 142.24) (angle -90) (layer Edge.Cuts) (width 0.1))
 (gr_arc (start 100.33 73.66) (end 100.33 68.58) (angle -90) (layer Edge.Cuts) (width 0.1))
 (gr_arc (start 100.33 137.16) (end 95.25 137.16) (angle -90) (layer Edge.Cuts) (width 0.1))
 (gr_line (start 100.33 142.24) (end 185.42 142.24) (layer Edge.Cuts) (width 0.1))
 (gr_line (start 95.25 73.66) (end 95.25 137.16) (layer Edge.Cuts) (width 0.1))
 (gr_line (start 185.42 68.58) (end 100.33 68.58) (layer Edge.Cuts) (width 0.1))
 (gr_line (start 190.5 137.16) (end 190.5 73.66) (layer Edge.Cuts) (width 0.1))
 (segment (start 120.65 81.32) (end 125.69 81.32) (width 0.5) (layer B.Cu) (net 3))
 (segment (start 125.73 81.28) (end 125.73 71.12) (width 0.5) (layer B.Cu) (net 3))
 (segment (start 125.69 81.32) (end 125.73 81.28) (width 0.5) (layer B.Cu) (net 3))
 (segment (start 146.05 71.12) (end 125.73 71.12) (width 0.5) (layer B.Cu) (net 3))
 (segment (start 111.76 88.9) (end 111.62 88.94) (width 0.5) (layer B.Cu) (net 3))
 (segment (start 161.29 81.28) (end 153.67 81.28) (width 0.5) (layer B.Cu) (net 3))
 (segment (start 148.59 71.12) (end 146.05 71.12) (width 0.5) (layer B.Cu) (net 3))
 (segment (start 148.59 81.28) (end 148.59 71.12) (width 0.5) (layer B.Cu) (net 3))
 (segment (start 151.13 83.82) (end 151.13 81.28) (width 0.5) (layer B.Cu) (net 3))
 (segment (start 153.67 81.28) (end 151.13 81.28) (width 0.5) (layer B.Cu) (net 3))
 (segment (start 151.13 81.28) (end 148.59 81.28) (width 0.5) (layer B.Cu) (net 3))
 (segment (start 111.76 88.9) (end 107.95 88.9) (width 0.5) (layer B.Cu) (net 3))
 (segment (start 107.95 88.9) (end 107.95 85.09) (width 0.5) (layer B.Cu) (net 3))
 (segment (start 120.65 81.32) (end 120.65 83.86) (width 0.5) (layer B.Cu) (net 3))
 (segment (start 107.95 85.09) (end 107.95 78.74) (width 0.5) (layer B.Cu) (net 3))
 (segment (start 176.53 88.9) (end 176.53 73.66) (width 0.5) (layer B.Cu) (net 3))
 (segment (start 107.95 83.82) (end 107.95 71.12) (width 0.5) (layer B.Cu) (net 3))
 (segment (start 120.65 83.86) (end 107.99 83.86) (width 0.5) (layer B.Cu) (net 3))
 (segment (start 107.99 83.86) (end 107.95 83.82) (width 0.5) (layer B.Cu) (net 3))
 (segment (start 107.95 71.12) (end 110.49 71.12) (width 0.5) (layer B.Cu) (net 3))
 (segment (start 118.11 88.9) (end 111.76 88.9) (width 0.5) (layer B.Cu) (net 3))
 (segment (start 138.43 86.36) (end 138.43 88.9) (width 0.5) (layer B.Cu) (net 3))
 (segment (start 138.43 88.9) (end 118.11 88.9) (width 0.5) (layer B.Cu) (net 3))
 (segment (start 151.13 83.82) (end 151.13 91.44) (width 0.5) (layer B.Cu) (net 3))
 (segment (start 151.13 91.44) (end 156.21 91.44) (width 0.5) (layer B.Cu) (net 3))
 (segment (start 176.53 91.44) (end 176.53 88.9) (width 0.5) (layer B.Cu) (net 3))
 (segment (start 158.75 91.28) (end 158.75 91.44) (width 0.5) (layer B.Cu) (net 3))
 (segment (start 156.21 91.44) (end 158.75 91.44) (width 0.5) (layer B.Cu) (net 3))
 (segment (start 161.14 91.29) (end 161.29 91.44) (width 0.5) (layer B.Cu) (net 3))
 (segment (start 161.14 90.86) (end 161.14 91.29) (width 0.5) (layer B.Cu) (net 3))
 (segment (start 158.75 91.44) (end 161.29 91.44) (width 0.5) (layer B.Cu) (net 3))
 (segment (start 167.64 90.86) (end 167.64 91.44) (width 0.5) (layer B.Cu) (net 3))
 (segment (start 161.29 91.44) (end 167.64 91.44) (width 0.5) (layer B.Cu) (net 3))
 (segment (start 167.64 91.44) (end 176.53 91.44) (width 0.5) (layer B.Cu) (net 3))
 (segment (start 161.29 76.2) (end 156.21 76.2) (width 0.25) (layer B.Cu) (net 17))
 (segment (start 156.21 76.2) (end 156.21 71.12) (width 0.25) (layer B.Cu) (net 17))
 (segment (start 153.71 78.74) (end 153.67 78.78) (width 0.25) (layer B.Cu) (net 19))
 (segment (start 161.29 78.74) (end 153.71 78.74) (width 0.25) (layer B.Cu) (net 19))
 (segment (start 151.33 71.12) (end 153.67 71.12) (width 0.25) (layer B.Cu) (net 19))
 (segment (start 153.67 71.12) (end 153.67 78.78) (width 0.25) (layer B.Cu) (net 19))
 (segment (start 146.05 88.9) (end 140.97 88.9) (width 0.5) (layer B.Cu) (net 18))
 (segment (start 140.97 83.82) (end 140.97 88.9) (width 0.5) (layer B.Cu) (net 18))
 (segment (start 148.59 88.9) (end 146.05 88.9) (width 0.5) (layer B.Cu) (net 18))
 (segment (start 148.63 88.94) (end 148.59 88.9) (width 0.5) (layer B.Cu) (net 18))
 (segment (start 148.63 91.44) (end 148.63 88.94) (width 0.5) (layer B.Cu) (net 18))
 (segment (start 138.43 91.44) (end 140.97 88.9) (width 0.5) (layer B.Cu) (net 18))
 (segment (start 105.41 91.44) (end 138.43 91.44) (width 0.5) (layer B.Cu) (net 18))
 (segment (start 128.27 81.28) (end 128.27 76.2) (width 0.5) (layer B.Cu) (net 14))
 (segment (start 130.81 78.74) (end 128.27 78.74) (width 0.5) (layer B.Cu) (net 14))
 (segment (start 123.19 86.2) (end 123.19 83.82) (width 0.5) (layer B.Cu) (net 13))
 (segment (start 128.27 86.36) (end 128.27 86.28) (width 0.5) (layer B.Cu) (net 13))
 (segment (start 110.49 86.36) (end 128.27 86.36) (width 0.5) (layer B.Cu) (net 13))
 (segment (start 110.45 81.32) (end 110.49 81.36) (width 0.5) (layer B.Cu) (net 12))
 (segment (start 110.45 78.74) (end 110.45 81.32) (width 0.5) (layer B.Cu) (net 12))
 (segment (start 112.95 81.36) (end 113.03 81.28) (width 0.5) (layer B.Cu) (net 12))
 (segment (start 110.49 81.36) (end 112.95 81.36) (width 0.5) (layer B.Cu) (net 12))
 (segment (start 115.57 76.2) (end 113.03 76.2) (width 0.5) (layer B.Cu) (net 12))
 (segment (start 113.03 81.28) (end 113.03 76.2) (width 0.5) (layer B.Cu) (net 12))
 (segment (start 113.03 76.2) (end 113.03 71.12) (width 0.5) (layer B.Cu) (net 12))
 (segment (start 168.91 71.12) (end 168.91 73.66) (width 0.25) (layer B.Cu) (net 15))
 (segment (start 168.91 73.66) (end 163.83 73.66) (width 0.25) (layer B.Cu) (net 15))
 (segment (start 168.91 71.12) (end 171.45 71.12) (width 0.25) (layer B.Cu) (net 15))
 (segment (start 153.67 88.9) (end 163.83 88.9) (width 0.25) (layer B.Cu) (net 15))
 (segment (start 163.83 88.9) (end 163.83 73.66) (width 0.25) (layer B.Cu) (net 15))
 (segment (start 171.45 88.9) (end 173.99 88.9) (width 0.25) (layer B.Cu) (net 11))
 (segment (start 171.45 81.28) (end 173.99 81.28) (width 0.25) (layer B.Cu) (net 9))
 (segment (start 171.45 73.66) (end 173.99 73.66) (width 0.25) (layer B.Cu) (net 22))
 (segment (start 161.29 71.12) (end 161.29 73.66) (width 0.25) (layer B.Cu) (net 16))
 (segment (start 168.91 83.82) (end 168.91 81.28) (width 0.25) (layer B.Cu) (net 10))
 (segment (start 168.91 83.82) (end 171.45 83.82) (width 0.25) (layer B.Cu) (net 10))
 (segment (start 120.65 73.66) (end 120.65 76.2) (width 0.5) (layer B.Cu) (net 20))
 (segment (start 123.19 73.66) (end 120.65 73.66) (width 0.5) (layer B.Cu) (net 20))
 (segment (start 168.91 76.2) (end 171.45 76.2) (width 0.25) (layer B.Cu) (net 8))
 (segment (start 168.91 78.74) (end 166.37 78.74) (width 0.25) (layer B.Cu) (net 4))
 (segment (start 166.37 78.74) (end 166.37 86.36) (width 0.25) (layer B.Cu) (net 4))
 (segment (start 166.37 86.36) (end 167.64 86.36) (width 0.25) (layer B.Cu) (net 4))
 (segment (start 161.14 86.36) (end 167.64 86.36) (width 0.25) (layer F.Cu) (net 4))
 (segment (start 115.57 71.12) (end 118.11 71.12) (width 0.5) (layer B.Cu) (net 21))
 (segment (start 118.11 71.12) (end 118.11 76.2) (width 0.5) (layer B.Cu) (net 21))
 (segment (start 143.51 73.66) (end 130.81 73.66) (width 0.25) (layer B.Cu) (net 6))
 (segment (start 143.51 83.82) (end 143.51 73.66) (width 0.25) (layer B.Cu) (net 6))
 (segment (start 161.29 83.82) (end 153.67 83.82) (width 0.25) (layer B.Cu) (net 6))
 (segment (start 143.51 83.82) (end 148.59 83.82) (width 0.25) (layer B.Cu) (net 6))
 (segment (start 153.67 83.82) (end 153.67 83.82) (width 0.25) (layer B.Cu) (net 6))
 (via (at 153.67 83.82) (size 0.8) (drill 0.4) (layers F.Cu B.Cu) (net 6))
 (segment (start 148.59 83.82) (end 148.59 83.82) (width 0.25) (layer B.Cu) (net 6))
 (via (at 148.59 83.82) (size 0.8) (drill 0.4) (layers F.Cu B.Cu) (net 6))
 (segment (start 133.35 78.74) (end 133.35 76.2) (width 0.5) (layer B.Cu) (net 5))
 (segment (start 133.35 76.2) (end 130.81 76.2) (width 0.5) (layer B.Cu) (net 5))
 (segment (start 138.43 83.82) (end 138.43 76.2) (width 0.5) (layer B.Cu) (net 5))
 (segment (start 140.97 76.2) (end 138.43 76.2) (width 0.5) (layer B.Cu) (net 5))
 (segment (start 138.43 76.2) (end 133.35 76.2) (width 0.5) (layer B.Cu) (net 5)))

